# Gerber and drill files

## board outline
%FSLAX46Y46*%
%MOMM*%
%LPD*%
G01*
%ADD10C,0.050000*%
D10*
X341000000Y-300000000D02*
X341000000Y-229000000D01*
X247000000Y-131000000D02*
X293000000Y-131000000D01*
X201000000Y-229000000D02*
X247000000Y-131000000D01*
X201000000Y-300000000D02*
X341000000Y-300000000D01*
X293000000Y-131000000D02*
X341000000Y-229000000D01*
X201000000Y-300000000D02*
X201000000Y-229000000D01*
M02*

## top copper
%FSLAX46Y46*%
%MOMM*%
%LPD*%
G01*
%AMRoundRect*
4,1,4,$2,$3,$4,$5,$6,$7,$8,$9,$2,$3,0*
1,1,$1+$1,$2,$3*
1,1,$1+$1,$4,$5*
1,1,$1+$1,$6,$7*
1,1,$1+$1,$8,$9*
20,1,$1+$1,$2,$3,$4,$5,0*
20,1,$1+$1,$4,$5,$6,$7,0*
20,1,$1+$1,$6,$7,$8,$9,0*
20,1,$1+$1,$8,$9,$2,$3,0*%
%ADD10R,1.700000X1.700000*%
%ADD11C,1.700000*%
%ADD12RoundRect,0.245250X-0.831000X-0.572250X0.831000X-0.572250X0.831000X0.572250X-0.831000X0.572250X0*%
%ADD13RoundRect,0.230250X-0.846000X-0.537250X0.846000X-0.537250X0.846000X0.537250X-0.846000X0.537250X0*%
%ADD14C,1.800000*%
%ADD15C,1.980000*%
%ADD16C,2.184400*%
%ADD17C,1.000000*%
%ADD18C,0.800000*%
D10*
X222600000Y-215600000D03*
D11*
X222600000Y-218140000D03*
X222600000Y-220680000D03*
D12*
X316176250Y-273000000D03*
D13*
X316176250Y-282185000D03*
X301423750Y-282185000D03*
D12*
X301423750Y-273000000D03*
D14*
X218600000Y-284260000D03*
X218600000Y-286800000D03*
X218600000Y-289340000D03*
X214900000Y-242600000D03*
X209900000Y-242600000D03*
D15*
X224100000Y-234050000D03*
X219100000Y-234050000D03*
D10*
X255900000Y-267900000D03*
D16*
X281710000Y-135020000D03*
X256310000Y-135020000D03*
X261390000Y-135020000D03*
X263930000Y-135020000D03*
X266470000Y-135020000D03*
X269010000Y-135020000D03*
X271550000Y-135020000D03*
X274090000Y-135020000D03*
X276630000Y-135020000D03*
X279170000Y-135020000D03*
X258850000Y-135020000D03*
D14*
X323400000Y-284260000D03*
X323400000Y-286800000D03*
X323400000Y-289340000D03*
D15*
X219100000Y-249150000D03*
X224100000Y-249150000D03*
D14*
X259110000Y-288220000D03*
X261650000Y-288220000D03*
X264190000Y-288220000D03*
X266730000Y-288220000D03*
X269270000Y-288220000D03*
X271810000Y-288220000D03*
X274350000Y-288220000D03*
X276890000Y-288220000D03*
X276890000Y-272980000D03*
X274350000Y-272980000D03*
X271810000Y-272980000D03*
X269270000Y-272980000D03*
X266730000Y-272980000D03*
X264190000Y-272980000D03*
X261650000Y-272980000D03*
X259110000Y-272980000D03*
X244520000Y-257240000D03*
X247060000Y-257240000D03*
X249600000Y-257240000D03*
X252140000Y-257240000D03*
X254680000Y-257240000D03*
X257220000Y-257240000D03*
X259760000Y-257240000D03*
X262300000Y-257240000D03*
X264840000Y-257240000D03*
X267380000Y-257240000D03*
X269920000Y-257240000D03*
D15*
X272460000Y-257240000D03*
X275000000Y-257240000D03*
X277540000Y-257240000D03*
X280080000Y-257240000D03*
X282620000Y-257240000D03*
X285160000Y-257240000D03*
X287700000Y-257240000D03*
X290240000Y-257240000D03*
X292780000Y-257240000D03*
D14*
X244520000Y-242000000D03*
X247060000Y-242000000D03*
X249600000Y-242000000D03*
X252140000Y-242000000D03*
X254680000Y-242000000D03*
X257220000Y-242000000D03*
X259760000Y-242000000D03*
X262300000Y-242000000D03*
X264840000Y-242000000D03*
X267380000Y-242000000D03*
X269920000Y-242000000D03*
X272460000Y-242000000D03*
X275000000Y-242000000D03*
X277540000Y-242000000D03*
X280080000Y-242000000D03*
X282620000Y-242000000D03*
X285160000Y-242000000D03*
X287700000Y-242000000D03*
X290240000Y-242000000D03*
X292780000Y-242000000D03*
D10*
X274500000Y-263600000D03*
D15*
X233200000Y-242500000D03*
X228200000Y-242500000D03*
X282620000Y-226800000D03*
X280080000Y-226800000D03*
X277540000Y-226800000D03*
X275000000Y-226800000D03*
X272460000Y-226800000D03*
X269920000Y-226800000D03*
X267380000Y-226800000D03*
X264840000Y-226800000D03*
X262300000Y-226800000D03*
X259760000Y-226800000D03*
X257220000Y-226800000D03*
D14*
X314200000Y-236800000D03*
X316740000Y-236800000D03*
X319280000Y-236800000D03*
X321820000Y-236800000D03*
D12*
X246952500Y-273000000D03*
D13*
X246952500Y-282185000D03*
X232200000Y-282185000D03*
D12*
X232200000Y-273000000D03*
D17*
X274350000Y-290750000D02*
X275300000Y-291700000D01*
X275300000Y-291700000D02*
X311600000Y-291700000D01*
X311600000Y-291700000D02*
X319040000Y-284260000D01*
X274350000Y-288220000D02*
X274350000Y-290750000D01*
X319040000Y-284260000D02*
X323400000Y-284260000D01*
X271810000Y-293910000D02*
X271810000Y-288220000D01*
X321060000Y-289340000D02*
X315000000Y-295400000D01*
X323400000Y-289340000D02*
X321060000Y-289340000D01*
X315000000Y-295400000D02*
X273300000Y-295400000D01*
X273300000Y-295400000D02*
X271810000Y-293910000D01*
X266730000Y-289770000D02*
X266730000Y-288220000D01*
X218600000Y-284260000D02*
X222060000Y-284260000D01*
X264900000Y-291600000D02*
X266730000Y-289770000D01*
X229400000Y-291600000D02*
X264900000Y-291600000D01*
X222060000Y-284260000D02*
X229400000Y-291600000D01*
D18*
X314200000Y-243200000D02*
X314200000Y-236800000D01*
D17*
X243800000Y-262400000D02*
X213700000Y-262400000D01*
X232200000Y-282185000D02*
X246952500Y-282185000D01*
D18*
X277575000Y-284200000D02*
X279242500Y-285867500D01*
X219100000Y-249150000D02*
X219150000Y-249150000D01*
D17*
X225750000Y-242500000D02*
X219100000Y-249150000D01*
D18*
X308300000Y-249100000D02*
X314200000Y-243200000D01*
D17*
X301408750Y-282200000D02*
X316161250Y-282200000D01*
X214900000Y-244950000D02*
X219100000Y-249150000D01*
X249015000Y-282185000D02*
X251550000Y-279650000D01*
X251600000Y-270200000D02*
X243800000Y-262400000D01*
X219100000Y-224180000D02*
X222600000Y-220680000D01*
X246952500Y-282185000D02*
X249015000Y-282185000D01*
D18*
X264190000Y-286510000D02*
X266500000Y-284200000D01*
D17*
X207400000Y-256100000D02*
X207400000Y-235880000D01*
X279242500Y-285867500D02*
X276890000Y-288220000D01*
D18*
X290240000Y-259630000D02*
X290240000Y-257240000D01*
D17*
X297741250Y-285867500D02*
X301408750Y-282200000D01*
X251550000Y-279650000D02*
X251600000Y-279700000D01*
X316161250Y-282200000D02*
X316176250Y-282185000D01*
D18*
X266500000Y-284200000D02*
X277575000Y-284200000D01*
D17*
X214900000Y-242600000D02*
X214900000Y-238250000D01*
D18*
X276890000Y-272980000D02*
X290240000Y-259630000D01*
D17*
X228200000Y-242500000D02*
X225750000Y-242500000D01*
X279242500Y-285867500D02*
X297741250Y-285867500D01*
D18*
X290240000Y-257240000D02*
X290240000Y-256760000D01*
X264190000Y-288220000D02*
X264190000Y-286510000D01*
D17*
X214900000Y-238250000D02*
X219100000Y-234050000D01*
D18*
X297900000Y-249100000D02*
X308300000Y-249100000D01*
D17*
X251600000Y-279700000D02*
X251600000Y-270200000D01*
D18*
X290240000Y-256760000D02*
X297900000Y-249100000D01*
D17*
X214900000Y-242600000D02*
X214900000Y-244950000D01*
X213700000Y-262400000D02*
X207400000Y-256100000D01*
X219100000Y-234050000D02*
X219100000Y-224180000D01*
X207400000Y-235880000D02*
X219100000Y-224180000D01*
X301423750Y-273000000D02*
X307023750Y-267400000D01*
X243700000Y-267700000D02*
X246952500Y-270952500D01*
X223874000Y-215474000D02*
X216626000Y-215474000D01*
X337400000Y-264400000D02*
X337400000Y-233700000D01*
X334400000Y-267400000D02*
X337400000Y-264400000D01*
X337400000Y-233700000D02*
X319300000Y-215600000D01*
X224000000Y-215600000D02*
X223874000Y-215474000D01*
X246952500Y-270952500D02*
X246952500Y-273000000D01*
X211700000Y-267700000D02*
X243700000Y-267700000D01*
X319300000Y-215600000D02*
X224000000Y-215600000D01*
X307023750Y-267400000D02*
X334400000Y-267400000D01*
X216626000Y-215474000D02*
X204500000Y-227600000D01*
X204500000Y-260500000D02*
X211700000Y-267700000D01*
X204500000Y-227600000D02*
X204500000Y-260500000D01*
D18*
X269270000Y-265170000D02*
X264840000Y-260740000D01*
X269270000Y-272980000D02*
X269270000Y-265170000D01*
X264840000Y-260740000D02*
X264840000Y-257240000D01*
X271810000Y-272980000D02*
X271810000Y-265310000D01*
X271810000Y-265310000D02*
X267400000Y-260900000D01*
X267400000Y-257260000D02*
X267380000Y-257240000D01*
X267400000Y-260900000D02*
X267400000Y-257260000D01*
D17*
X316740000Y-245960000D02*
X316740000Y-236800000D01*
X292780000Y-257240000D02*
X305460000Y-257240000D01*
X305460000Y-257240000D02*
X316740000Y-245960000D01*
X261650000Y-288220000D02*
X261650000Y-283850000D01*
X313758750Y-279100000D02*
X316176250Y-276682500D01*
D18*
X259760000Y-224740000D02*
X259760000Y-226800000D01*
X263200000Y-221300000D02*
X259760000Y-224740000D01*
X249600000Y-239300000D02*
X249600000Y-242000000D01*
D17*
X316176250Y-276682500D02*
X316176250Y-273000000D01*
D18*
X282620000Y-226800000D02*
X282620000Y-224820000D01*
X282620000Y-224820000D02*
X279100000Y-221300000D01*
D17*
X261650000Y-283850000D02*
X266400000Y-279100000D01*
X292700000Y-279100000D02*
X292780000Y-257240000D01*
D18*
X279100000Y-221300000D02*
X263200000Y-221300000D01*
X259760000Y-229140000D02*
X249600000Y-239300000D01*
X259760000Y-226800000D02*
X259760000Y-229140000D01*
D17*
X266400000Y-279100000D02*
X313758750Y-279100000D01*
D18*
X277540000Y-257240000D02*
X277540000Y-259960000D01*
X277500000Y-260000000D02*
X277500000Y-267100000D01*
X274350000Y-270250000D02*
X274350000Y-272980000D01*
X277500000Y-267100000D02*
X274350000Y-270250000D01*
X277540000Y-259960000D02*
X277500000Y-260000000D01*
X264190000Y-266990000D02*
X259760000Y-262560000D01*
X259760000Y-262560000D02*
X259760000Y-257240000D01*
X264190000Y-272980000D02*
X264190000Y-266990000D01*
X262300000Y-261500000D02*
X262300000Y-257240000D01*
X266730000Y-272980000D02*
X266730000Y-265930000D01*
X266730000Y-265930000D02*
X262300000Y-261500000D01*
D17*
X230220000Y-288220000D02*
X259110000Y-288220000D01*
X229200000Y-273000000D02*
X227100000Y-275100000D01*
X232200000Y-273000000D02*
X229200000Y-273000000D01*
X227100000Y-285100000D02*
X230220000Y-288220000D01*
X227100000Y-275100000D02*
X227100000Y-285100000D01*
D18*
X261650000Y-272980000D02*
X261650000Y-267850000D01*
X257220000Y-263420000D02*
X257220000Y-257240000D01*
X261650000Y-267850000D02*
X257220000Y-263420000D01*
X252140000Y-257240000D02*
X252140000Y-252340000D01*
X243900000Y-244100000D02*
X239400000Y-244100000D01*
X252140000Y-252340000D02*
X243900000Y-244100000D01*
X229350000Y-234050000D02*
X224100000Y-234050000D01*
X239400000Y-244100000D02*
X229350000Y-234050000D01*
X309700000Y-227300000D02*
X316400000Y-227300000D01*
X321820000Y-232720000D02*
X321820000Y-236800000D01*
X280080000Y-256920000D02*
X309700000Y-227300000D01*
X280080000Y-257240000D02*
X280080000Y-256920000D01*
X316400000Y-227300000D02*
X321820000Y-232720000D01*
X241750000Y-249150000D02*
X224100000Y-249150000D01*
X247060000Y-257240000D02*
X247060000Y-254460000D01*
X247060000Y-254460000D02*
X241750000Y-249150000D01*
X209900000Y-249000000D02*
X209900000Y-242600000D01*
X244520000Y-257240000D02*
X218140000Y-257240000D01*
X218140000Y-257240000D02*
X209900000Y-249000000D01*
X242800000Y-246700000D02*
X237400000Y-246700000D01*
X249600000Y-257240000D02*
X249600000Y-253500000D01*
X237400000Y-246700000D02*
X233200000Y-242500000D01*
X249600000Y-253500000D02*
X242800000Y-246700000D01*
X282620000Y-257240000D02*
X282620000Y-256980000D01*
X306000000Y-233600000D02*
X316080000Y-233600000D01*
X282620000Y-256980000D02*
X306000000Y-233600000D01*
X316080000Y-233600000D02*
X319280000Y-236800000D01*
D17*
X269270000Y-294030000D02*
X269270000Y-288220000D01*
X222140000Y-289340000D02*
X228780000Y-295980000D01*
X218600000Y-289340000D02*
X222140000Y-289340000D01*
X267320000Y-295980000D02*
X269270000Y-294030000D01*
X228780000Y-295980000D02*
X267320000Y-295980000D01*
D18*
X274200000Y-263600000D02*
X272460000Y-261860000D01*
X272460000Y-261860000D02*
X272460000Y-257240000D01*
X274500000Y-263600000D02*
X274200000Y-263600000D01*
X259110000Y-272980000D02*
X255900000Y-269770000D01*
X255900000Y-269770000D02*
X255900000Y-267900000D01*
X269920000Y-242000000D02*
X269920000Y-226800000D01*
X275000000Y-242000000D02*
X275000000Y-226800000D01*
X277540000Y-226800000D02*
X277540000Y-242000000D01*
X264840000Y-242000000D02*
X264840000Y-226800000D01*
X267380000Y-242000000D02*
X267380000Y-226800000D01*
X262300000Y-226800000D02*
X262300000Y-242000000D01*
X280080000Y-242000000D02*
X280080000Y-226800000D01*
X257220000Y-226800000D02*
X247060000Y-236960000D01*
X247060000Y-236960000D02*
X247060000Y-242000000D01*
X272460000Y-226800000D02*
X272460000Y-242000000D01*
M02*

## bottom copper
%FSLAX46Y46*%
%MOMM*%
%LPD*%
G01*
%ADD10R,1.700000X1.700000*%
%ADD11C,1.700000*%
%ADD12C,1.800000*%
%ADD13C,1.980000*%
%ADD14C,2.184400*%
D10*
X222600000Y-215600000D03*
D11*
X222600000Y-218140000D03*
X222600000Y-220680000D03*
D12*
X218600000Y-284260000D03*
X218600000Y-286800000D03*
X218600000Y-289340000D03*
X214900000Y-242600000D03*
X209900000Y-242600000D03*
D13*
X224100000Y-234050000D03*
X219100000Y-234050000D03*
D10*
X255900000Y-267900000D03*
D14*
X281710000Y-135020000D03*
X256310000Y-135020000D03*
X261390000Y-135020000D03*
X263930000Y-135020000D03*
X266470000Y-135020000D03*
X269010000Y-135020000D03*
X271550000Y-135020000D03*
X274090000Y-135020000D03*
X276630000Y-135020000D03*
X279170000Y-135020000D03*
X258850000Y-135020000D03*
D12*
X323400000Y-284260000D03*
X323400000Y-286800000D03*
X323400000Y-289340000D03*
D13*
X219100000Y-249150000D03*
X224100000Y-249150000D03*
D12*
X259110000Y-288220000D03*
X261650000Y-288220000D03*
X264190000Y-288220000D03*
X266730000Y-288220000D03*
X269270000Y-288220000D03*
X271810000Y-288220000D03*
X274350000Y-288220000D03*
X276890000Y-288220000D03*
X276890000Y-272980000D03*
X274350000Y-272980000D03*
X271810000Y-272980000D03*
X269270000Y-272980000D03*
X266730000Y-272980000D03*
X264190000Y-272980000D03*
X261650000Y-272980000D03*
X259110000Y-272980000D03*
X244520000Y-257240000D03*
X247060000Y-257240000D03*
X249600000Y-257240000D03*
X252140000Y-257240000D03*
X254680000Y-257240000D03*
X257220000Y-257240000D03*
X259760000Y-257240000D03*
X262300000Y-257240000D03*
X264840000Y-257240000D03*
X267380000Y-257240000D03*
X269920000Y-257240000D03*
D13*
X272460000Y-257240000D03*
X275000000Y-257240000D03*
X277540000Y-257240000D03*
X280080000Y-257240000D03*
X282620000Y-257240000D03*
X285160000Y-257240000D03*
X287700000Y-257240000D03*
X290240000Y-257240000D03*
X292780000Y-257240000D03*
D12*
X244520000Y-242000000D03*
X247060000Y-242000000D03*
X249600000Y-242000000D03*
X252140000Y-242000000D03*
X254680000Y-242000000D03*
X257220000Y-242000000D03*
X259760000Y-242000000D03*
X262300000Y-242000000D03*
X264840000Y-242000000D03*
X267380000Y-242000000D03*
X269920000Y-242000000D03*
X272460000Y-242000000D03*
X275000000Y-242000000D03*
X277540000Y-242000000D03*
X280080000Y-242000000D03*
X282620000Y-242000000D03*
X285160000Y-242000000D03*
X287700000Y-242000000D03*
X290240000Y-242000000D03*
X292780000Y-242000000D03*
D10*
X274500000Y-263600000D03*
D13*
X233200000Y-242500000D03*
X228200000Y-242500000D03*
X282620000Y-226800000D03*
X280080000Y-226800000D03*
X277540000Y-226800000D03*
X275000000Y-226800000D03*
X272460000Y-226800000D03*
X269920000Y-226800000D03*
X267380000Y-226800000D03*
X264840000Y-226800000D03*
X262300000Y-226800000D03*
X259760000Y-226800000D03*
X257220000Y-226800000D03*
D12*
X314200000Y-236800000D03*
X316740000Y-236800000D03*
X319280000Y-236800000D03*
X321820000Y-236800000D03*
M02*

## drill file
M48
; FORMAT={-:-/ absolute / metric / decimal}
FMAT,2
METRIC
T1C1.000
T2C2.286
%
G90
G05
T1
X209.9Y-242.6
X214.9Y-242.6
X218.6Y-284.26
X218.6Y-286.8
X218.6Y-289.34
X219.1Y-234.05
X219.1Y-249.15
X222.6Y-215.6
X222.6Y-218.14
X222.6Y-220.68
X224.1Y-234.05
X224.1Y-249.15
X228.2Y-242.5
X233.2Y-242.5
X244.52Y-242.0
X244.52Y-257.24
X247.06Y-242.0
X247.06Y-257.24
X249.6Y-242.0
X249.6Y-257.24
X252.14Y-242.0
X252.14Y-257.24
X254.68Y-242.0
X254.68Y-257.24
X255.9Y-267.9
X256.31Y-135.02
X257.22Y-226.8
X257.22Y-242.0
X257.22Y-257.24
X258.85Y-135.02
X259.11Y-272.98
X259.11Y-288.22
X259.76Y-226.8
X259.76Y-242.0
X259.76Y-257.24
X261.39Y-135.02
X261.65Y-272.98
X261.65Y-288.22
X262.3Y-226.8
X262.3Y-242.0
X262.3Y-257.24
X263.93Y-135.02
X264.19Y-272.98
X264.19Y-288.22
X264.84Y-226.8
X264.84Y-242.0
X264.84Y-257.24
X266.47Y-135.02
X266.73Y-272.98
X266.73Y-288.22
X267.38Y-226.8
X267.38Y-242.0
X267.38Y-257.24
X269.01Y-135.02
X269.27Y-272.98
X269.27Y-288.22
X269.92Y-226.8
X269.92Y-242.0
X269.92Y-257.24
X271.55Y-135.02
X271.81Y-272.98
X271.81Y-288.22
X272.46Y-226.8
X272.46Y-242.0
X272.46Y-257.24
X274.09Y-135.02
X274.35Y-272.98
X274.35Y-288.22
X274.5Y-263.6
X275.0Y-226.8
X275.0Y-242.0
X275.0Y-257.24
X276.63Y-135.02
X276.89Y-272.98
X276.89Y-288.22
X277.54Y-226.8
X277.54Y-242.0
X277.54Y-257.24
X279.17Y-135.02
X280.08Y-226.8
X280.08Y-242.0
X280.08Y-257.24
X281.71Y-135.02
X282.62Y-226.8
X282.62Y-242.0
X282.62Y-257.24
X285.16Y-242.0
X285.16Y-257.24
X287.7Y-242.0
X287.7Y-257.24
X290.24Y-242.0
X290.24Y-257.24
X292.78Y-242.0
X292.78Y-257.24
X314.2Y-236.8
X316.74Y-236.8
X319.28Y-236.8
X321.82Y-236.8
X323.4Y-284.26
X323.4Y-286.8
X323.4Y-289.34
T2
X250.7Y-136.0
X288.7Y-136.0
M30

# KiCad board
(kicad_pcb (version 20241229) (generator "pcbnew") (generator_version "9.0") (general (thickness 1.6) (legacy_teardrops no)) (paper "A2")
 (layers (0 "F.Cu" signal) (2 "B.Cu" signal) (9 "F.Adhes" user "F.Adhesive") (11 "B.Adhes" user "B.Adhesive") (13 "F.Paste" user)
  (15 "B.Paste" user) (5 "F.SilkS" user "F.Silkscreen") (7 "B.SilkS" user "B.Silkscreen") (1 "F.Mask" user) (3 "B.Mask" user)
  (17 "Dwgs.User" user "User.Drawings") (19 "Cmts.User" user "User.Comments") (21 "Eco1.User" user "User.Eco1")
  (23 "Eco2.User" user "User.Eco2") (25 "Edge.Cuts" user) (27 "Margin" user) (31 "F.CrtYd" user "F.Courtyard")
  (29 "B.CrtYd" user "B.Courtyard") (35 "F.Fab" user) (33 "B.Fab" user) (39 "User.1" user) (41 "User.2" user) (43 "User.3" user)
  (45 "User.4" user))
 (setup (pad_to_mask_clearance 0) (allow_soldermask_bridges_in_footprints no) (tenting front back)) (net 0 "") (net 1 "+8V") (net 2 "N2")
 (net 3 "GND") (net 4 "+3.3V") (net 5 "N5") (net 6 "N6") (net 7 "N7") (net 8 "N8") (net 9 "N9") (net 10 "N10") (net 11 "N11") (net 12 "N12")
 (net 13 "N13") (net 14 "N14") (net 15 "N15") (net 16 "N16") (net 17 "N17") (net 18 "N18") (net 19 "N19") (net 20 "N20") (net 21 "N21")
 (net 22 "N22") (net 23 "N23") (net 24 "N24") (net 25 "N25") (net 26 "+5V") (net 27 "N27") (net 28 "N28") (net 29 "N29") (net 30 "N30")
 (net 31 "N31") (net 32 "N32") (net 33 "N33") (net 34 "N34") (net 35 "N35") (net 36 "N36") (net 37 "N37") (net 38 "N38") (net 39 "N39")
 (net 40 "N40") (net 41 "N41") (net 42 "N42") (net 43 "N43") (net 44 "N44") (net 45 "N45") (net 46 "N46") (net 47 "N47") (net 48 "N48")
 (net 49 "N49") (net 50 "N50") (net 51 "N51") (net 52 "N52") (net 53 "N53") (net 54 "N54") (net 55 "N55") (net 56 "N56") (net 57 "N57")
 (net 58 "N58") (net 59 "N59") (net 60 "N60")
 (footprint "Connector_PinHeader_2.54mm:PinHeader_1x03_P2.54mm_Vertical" (layer "F.Cu") (at 222.6 215.6)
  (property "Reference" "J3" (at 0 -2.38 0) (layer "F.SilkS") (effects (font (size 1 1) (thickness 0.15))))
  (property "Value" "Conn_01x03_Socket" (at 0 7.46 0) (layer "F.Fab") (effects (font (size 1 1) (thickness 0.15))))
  (pad "1" thru_hole rect (at 0 0) (size 1.7 1.7) (drill 1) (layers "*.Cu" "*.Mask") (remove_unused_layers no) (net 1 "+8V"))
  (pad "2" thru_hole circle (at 0 2.54) (size 1.7 1.7) (drill 1) (layers "*.Cu" "*.Mask") (remove_unused_layers no) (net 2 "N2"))
  (pad "3" thru_hole circle (at 0 5.08) (size 1.7 1.7) (drill 1) (layers "*.Cu" "*.Mask") (remove_unused_layers no) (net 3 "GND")))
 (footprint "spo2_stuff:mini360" (layer "F.Cu") (at 308.8 277.5175)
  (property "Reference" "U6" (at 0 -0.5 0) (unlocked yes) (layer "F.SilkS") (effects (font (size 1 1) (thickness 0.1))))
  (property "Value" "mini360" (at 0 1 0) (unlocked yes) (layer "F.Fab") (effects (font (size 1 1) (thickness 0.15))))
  (pad "1" smd roundrect (at 7.37625 -4.5175) (size 2.1525 1.635) (layers "F.Cu" "F.Mask" "F.Paste") (roundrect_rratio 0.15) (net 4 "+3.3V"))
  (pad "2" smd roundrect (at 7.37625 4.6675) (size 2.1525 1.535) (layers "F.Cu" "F.Mask" "F.Paste") (roundrect_rratio 0.15) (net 3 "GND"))
  (pad "3" smd roundrect (at -7.37625 4.6675) (size 2.1525 1.535) (layers "F.Cu" "F.Mask" "F.Paste") (roundrect_rratio 0.15) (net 3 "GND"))
  (pad "4" smd roundrect (at -7.37625 -4.5175) (size 2.1525 1.635) (layers "F.Cu" "F.Mask" "F.Paste") (roundrect_rratio 0.15) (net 1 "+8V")))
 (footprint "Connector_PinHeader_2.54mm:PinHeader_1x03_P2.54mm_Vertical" (layer "F.Cu") (at 218.6 284.26)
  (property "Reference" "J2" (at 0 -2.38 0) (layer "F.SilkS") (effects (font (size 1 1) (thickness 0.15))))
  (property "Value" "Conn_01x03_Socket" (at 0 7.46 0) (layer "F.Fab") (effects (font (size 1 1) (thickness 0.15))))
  (pad "1" thru_hole circle (at 0 0) (size 1.8 1.8) (drill 1) (layers "*.Cu" "*.Mask") (remove_unused_layers no) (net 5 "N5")
   (solder_mask_margin 0.102))
  (pad "2" thru_hole circle (at 0 2.54) (size 1.8 1.8) (drill 1) (layers "*.Cu" "*.Mask") (remove_unused_layers no) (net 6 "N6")
   (solder_mask_margin 0.102))
  (pad "3" thru_hole circle (at 0 5.08) (size 1.8 1.8) (drill 1) (layers "*.Cu" "*.Mask") (remove_unused_layers no) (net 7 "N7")
   (solder_mask_margin 0.102)))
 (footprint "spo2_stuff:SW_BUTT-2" (layer "F.Cu") (at 212.4 242.6 180)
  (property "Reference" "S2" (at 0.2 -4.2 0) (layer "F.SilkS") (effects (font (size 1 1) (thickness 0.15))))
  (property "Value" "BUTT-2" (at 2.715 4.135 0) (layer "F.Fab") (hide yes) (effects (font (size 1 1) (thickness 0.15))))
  (pad "1" thru_hole circle (at -2.5 0 180) (size 1.8 1.8) (drill 1) (layers "*.Cu" "*.Mask") (remove_unused_layers no) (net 3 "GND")
   (solder_mask_margin 0.102))
  (pad "2" thru_hole circle (at 2.5 0 180) (size 1.8 1.8) (drill 1) (layers "*.Cu" "*.Mask") (remove_unused_layers no) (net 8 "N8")
   (solder_mask_margin 0.102)))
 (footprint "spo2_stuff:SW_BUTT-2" (layer "F.Cu") (at 221.6 234.05 180)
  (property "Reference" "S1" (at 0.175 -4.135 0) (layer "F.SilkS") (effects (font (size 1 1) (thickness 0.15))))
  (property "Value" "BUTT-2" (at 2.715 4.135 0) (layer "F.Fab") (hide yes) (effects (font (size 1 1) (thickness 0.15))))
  (pad "1" thru_hole circle (at -2.5 0 180) (size 1.98 1.98) (drill 1) (layers "*.Cu" "*.Mask") (remove_unused_layers no) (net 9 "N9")
   (solder_mask_margin 0.102))
  (pad "2" thru_hole circle (at 2.5 0 180) (size 1.98 1.98) (drill 1) (layers "*.Cu" "*.Mask") (remove_unused_layers no) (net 3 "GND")
   (solder_mask_margin 0.102)))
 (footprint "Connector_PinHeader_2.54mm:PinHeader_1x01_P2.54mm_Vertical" (layer "F.Cu") (at 255.9 267.9)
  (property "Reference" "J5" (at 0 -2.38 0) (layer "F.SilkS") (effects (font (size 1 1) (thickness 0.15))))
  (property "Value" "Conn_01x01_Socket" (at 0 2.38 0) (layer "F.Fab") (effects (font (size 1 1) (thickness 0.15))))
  (pad "1" thru_hole rect (at 0 0) (size 1.7 1.7) (drill 1) (layers "*.Cu" "*.Mask") (remove_unused_layers no) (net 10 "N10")))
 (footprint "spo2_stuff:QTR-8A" (layer "F.Cu") (at 289.35 133.75)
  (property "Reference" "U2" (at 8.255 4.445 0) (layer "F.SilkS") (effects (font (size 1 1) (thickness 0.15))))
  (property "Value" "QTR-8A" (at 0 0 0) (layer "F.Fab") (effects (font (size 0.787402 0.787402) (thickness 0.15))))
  (pad "" np_thru_hole circle (at -38.65 2.25) (size 2.286 2.286) (drill 2.286) (layers "*.Cu" "*.Mask"))
  (pad "" np_thru_hole circle (at -0.65 2.25) (size 2.286 2.286) (drill 2.286) (layers "*.Cu" "*.Mask"))
  (pad "3V3" thru_hole circle (at -7.64 1.27) (size 2.1844 2.1844) (drill 1) (layers "*.Cu" "*.Mask") (remove_unused_layers no)
   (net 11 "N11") (solder_mask_margin 0.102))
  (pad "GND" thru_hole circle (at -33.04 1.27) (size 2.1844 2.1844) (drill 1) (layers "*.Cu" "*.Mask") (remove_unused_layers no)
   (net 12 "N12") (solder_mask_margin 0.102))
  (pad "LED1" thru_hole circle (at -27.96 1.27) (size 2.1844 2.1844) (drill 1) (layers "*.Cu" "*.Mask") (remove_unused_layers no)
   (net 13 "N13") (solder_mask_margin 0.102))
  (pad "LED2" thru_hole circle (at -25.42 1.27) (size 2.1844 2.1844) (drill 1) (layers "*.Cu" "*.Mask") (remove_unused_layers no)
   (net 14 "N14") (solder_mask_margin 0.102))
  (pad "LED3" thru_hole circle (at -22.88 1.27) (size 2.1844 2.1844) (drill 1) (layers "*.Cu" "*.Mask") (remove_unused_layers no)
   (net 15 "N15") (solder_mask_margin 0.102))
  (pad "LED4" thru_hole circle (at -20.34 1.27) (size 2.1844 2.1844) (drill 1) (layers "*.Cu" "*.Mask") (remove_unused_layers no)
   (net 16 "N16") (solder_mask_margin 0.102))
  (pad "LED5" thru_hole circle (at -17.8 1.27) (size 2.1844 2.1844) (drill 1) (layers "*.Cu" "*.Mask") (remove_unused_layers no)
   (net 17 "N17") (solder_mask_margin 0.102))
  (pad "LED6" thru_hole circle (at -15.26 1.27) (size 2.1844 2.1844) (drill 1) (layers "*.Cu" "*.Mask") (remove_unused_layers no)
   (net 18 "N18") (solder_mask_margin 0.102))
  (pad "LED7" thru_hole circle (at -12.72 1.27) (size 2.1844 2.1844) (drill 1) (layers "*.Cu" "*.Mask") (remove_unused_layers no)
   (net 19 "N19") (solder_mask_margin 0.102))
  (pad "LED8" thru_hole circle (at -10.18 1.27) (size 2.1844 2.1844) (drill 1) (layers "*.Cu" "*.Mask") (remove_unused_layers no)
   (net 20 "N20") (solder_mask_margin 0.102))
  (pad "LED_ON" thru_hole circle (at -30.5 1.27) (size 2.1844 2.1844) (drill 1) (layers "*.Cu" "*.Mask") (remove_unused_layers no)
   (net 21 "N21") (solder_mask_margin 0.102)))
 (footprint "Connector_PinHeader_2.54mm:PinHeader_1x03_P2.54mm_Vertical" (layer "F.Cu") (at 323.4 284.26)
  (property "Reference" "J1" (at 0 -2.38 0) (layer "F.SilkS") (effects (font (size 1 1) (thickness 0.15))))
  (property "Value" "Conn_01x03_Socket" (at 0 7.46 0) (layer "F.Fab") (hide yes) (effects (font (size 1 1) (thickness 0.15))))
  (pad "1" thru_hole circle (at 0 0) (size 1.8 1.8) (drill 1) (layers "*.Cu" "*.Mask") (remove_unused_layers no) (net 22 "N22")
   (solder_mask_margin 0.102))
  (pad "2" thru_hole circle (at 0 2.54) (size 1.8 1.8) (drill 1) (layers "*.Cu" "*.Mask") (remove_unused_layers no) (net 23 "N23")
   (solder_mask_margin 0.102))
  (pad "3" thru_hole circle (at 0 5.08) (size 1.8 1.8) (drill 1) (layers "*.Cu" "*.Mask") (remove_unused_layers no) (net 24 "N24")
   (solder_mask_margin 0.102)))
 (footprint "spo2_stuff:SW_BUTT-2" (layer "F.Cu") (at 221.6 249.15)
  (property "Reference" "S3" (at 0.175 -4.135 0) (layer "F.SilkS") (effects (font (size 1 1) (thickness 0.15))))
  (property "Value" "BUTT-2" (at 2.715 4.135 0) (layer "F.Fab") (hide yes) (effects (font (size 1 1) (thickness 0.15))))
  (pad "1" thru_hole circle (at -2.5 0) (size 1.98 1.98) (drill 1) (layers "*.Cu" "*.Mask") (remove_unused_layers no) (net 3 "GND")
   (solder_mask_margin 0.102))
  (pad "2" thru_hole circle (at 2.5 0) (size 1.98 1.98) (drill 1) (layers "*.Cu" "*.Mask") (remove_unused_layers no) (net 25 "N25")
   (solder_mask_margin 0.102)))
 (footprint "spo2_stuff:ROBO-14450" (layer "F.Cu") (at 268 280.6 90)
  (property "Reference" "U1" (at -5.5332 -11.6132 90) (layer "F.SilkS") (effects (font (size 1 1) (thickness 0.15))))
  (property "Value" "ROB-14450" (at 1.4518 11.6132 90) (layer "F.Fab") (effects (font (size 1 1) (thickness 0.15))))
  (pad "1" thru_hole circle (at -7.62 -8.89 90) (size 1.8 1.8) (drill 1) (layers "*.Cu" "*.Mask") (remove_unused_layers no) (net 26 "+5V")
   (solder_mask_margin 0.102))
  (pad "2" thru_hole circle (at -7.62 -6.35 90) (size 1.8 1.8) (drill 1) (layers "*.Cu" "*.Mask") (remove_unused_layers no) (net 4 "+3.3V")
   (solder_mask_margin 0.102))
  (pad "3" thru_hole circle (at -7.62 -3.81 90) (size 1.8 1.8) (drill 1) (layers "*.Cu" "*.Mask") (remove_unused_layers no) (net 3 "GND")
   (solder_mask_margin 0.102))
  (pad "4" thru_hole circle (at -7.62 -1.27 90) (size 1.8 1.8) (drill 1) (layers "*.Cu" "*.Mask") (remove_unused_layers no) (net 5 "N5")
   (solder_mask_margin 0.102))
  (pad "5" thru_hole circle (at -7.62 1.27 90) (size 1.8 1.8) (drill 1) (layers "*.Cu" "*.Mask") (remove_unused_layers no) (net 7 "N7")
   (solder_mask_margin 0.102))
  (pad "6" thru_hole circle (at -7.62 3.81 90) (size 1.8 1.8) (drill 1) (layers "*.Cu" "*.Mask") (remove_unused_layers no) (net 24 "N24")
   (solder_mask_margin 0.102))
  (pad "7" thru_hole circle (at -7.62 6.35 90) (size 1.8 1.8) (drill 1) (layers "*.Cu" "*.Mask") (remove_unused_layers no) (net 22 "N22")
   (solder_mask_margin 0.102))
  (pad "8" thru_hole circle (at -7.62 8.89 90) (size 1.8 1.8) (drill 1) (layers "*.Cu" "*.Mask") (remove_unused_layers no) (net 3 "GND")
   (solder_mask_margin 0.102))
  (pad "9" thru_hole circle (at 7.62 8.89 90) (size 1.8 1.8) (drill 1) (layers "*.Cu" "*.Mask") (remove_unused_layers no) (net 3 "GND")
   (solder_mask_margin 0.102))
  (pad "10" thru_hole circle (at 7.62 6.35 90) (size 1.8 1.8) (drill 1) (layers "*.Cu" "*.Mask") (remove_unused_layers no) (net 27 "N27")
   (solder_mask_margin 0.102))
  (pad "11" thru_hole circle (at 7.62 3.81 90) (size 1.8 1.8) (drill 1) (layers "*.Cu" "*.Mask") (remove_unused_layers no) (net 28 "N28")
   (solder_mask_margin 0.102))
  (pad "12" thru_hole circle (at 7.62 1.27 90) (size 1.8 1.8) (drill 1) (layers "*.Cu" "*.Mask") (remove_unused_layers no) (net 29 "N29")
   (solder_mask_margin 0.102))
  (pad "13" thru_hole circle (at 7.62 -1.27 90) (size 1.8 1.8) (drill 1) (layers "*.Cu" "*.Mask") (remove_unused_layers no) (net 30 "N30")
   (solder_mask_margin 0.102))
  (pad "14" thru_hole circle (at 7.62 -3.81 90) (size 1.8 1.8) (drill 1) (layers "*.Cu" "*.Mask") (remove_unused_layers no) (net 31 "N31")
   (solder_mask_margin 0.102))
  (pad "15" thru_hole circle (at 7.62 -6.35 90) (size 1.8 1.8) (drill 1) (layers "*.Cu" "*.Mask") (remove_unused_layers no) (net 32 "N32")
   (solder_mask_margin 0.102))
  (pad "16" thru_hole circle (at 7.62 -8.89 90) (size 1.8 1.8) (drill 1) (layers "*.Cu" "*.Mask") (remove_unused_layers no) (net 10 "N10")
   (solder_mask_margin 0.102)))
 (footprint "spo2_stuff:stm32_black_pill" (layer "F.Cu") (at 295.1 260.15 90)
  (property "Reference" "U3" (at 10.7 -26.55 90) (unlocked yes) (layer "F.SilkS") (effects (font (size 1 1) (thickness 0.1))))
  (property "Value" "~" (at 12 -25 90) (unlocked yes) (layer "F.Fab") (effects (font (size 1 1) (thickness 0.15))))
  (pad "1" thru_hole circle (at 2.91 -50.58 90) (size 1.8 1.8) (drill 1) (layers "*.Cu" "*.Mask") (remove_unused_layers no) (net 8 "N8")
   (solder_mask_margin 0.102))
  (pad "2" thru_hole circle (at 2.91 -48.04 90) (size 1.8 1.8) (drill 1) (layers "*.Cu" "*.Mask") (remove_unused_layers no) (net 25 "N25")
   (solder_mask_margin 0.102))
  (pad "3" thru_hole circle (at 2.91 -45.5 90) (size 1.8 1.8) (drill 1) (layers "*.Cu" "*.Mask") (remove_unused_layers no) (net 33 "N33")
   (solder_mask_margin 0.102))
  (pad "4" thru_hole circle (at 2.91 -42.96 90) (size 1.8 1.8) (drill 1) (layers "*.Cu" "*.Mask") (remove_unused_layers no) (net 9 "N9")
   (solder_mask_margin 0.102))
  (pad "5" thru_hole circle (at 2.91 -40.42 90) (size 1.8 1.8) (drill 1) (layers "*.Cu" "*.Mask") (remove_unused_layers no) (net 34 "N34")
   (solder_mask_margin 0.102))
  (pad "6" thru_hole circle (at 2.91 -37.88 90) (size 1.8 1.8) (drill 1) (layers "*.Cu" "*.Mask") (remove_unused_layers no) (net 32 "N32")
   (solder_mask_margin 0.102))
  (pad "7" thru_hole circle (at 2.91 -35.34 90) (size 1.8 1.8) (drill 1) (layers "*.Cu" "*.Mask") (remove_unused_layers no) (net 31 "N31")
   (solder_mask_margin 0.102))
  (pad "8" thru_hole circle (at 2.91 -32.8 90) (size 1.8 1.8) (drill 1) (layers "*.Cu" "*.Mask") (remove_unused_layers no) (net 30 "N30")
   (solder_mask_margin 0.102))
  (pad "9" thru_hole circle (at 2.91 -30.26 90) (size 1.8 1.8) (drill 1) (layers "*.Cu" "*.Mask") (remove_unused_layers no) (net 29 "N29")
   (solder_mask_margin 0.102))
  (pad "10" thru_hole circle (at 2.91 -27.72 90) (size 1.8 1.8) (drill 1) (layers "*.Cu" "*.Mask") (remove_unused_layers no) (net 28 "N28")
   (solder_mask_margin 0.102))
  (pad "11" thru_hole circle (at 2.91 -25.18 90) (size 1.8 1.8) (drill 1) (layers "*.Cu" "*.Mask") (remove_unused_layers no) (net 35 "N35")
   (solder_mask_margin 0.102))
  (pad "12" thru_hole circle (at 2.91 -22.64 90) (size 1.98 1.98) (drill 1) (layers "*.Cu" "*.Mask") (remove_unused_layers no)
   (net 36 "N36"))
  (pad "13" thru_hole circle (at 2.91 -20.1 90) (size 1.98 1.98) (drill 1) (layers "*.Cu" "*.Mask") (remove_unused_layers no) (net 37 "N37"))
  (pad "14" thru_hole circle (at 2.91 -17.56 90) (size 1.98 1.98) (drill 1) (layers "*.Cu" "*.Mask") (remove_unused_layers no)
   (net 27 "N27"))
  (pad "15" thru_hole circle (at 2.91 -15.02 90) (size 1.98 1.98) (drill 1) (layers "*.Cu" "*.Mask") (remove_unused_layers no)
   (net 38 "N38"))
  (pad "16" thru_hole circle (at 2.91 -12.48 90) (size 1.98 1.98) (drill 1) (layers "*.Cu" "*.Mask") (remove_unused_layers no)
   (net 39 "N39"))
  (pad "17" thru_hole circle (at 2.91 -9.94 90) (size 1.98 1.98) (drill 1) (layers "*.Cu" "*.Mask") (remove_unused_layers no) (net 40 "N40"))
  (pad "18" thru_hole circle (at 2.91 -7.4 90) (size 1.98 1.98) (drill 1) (layers "*.Cu" "*.Mask") (remove_unused_layers no) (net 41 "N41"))
  (pad "19" thru_hole circle (at 2.91 -4.86 90) (size 1.98 1.98) (drill 1) (layers "*.Cu" "*.Mask") (remove_unused_layers no) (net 3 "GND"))
  (pad "20" thru_hole circle (at 2.91 -2.32 90) (size 1.98 1.98) (drill 1) (layers "*.Cu" "*.Mask") (remove_unused_layers no)
   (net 4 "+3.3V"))
  (pad "21" thru_hole circle (at 18.15 -50.58 90) (size 1.8 1.8) (drill 1) (layers "*.Cu" "*.Mask") (remove_unused_layers no) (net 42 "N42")
   (solder_mask_margin 0.102))
  (pad "22" thru_hole circle (at 18.15 -48.04 90) (size 1.8 1.8) (drill 1) (layers "*.Cu" "*.Mask") (remove_unused_layers no) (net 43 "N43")
   (solder_mask_margin 0.102))
  (pad "23" thru_hole circle (at 18.15 -45.5 90) (size 1.8 1.8) (drill 1) (layers "*.Cu" "*.Mask") (remove_unused_layers no) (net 4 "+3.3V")
   (solder_mask_margin 0.102))
  (pad "24" thru_hole circle (at 18.15 -42.96 90) (size 1.8 1.8) (drill 1) (layers "*.Cu" "*.Mask") (remove_unused_layers no) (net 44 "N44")
   (solder_mask_margin 0.102))
  (pad "25" thru_hole circle (at 18.15 -40.42 90) (size 1.8 1.8) (drill 1) (layers "*.Cu" "*.Mask") (remove_unused_layers no) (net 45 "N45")
   (solder_mask_margin 0.102))
  (pad "26" thru_hole circle (at 18.15 -37.88 90) (size 1.8 1.8) (drill 1) (layers "*.Cu" "*.Mask") (remove_unused_layers no) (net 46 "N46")
   (solder_mask_margin 0.102))
  (pad "27" thru_hole circle (at 18.15 -35.34 90) (size 1.8 1.8) (drill 1) (layers "*.Cu" "*.Mask") (remove_unused_layers no) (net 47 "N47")
   (solder_mask_margin 0.102))
  (pad "28" thru_hole circle (at 18.15 -32.8 90) (size 1.8 1.8) (drill 1) (layers "*.Cu" "*.Mask") (remove_unused_layers no) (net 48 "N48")
   (solder_mask_margin 0.102))
  (pad "29" thru_hole circle (at 18.15 -30.26 90) (size 1.8 1.8) (drill 1) (layers "*.Cu" "*.Mask") (remove_unused_layers no) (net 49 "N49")
   (solder_mask_margin 0.102))
  (pad "30" thru_hole circle (at 18.15 -27.72 90) (size 1.8 1.8) (drill 1) (layers "*.Cu" "*.Mask") (remove_unused_layers no) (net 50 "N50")
   (solder_mask_margin 0.102))
  (pad "31" thru_hole circle (at 18.15 -25.18 90) (size 1.8 1.8) (drill 1) (layers "*.Cu" "*.Mask") (remove_unused_layers no) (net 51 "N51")
   (solder_mask_margin 0.102))
  (pad "32" thru_hole circle (at 18.15 -22.64 90) (size 1.8 1.8) (drill 1) (layers "*.Cu" "*.Mask") (remove_unused_layers no) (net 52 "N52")
   (solder_mask_margin 0.102))
  (pad "33" thru_hole circle (at 18.15 -20.1 90) (size 1.8 1.8) (drill 1) (layers "*.Cu" "*.Mask") (remove_unused_layers no) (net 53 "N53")
   (solder_mask_margin 0.102))
  (pad "34" thru_hole circle (at 18.15 -17.56 90) (size 1.8 1.8) (drill 1) (layers "*.Cu" "*.Mask") (remove_unused_layers no) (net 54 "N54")
   (solder_mask_margin 0.102))
  (pad "35" thru_hole circle (at 18.15 -15.02 90) (size 1.8 1.8) (drill 1) (layers "*.Cu" "*.Mask") (remove_unused_layers no) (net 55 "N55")
   (solder_mask_margin 0.102))
  (pad "36" thru_hole circle (at 18.15 -12.48 90) (size 1.8 1.8) (drill 1) (layers "*.Cu" "*.Mask") (remove_unused_layers no) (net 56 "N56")
   (solder_mask_margin 0.102))
  (pad "37" thru_hole circle (at 18.15 -9.94 90) (size 1.8 1.8) (drill 1) (layers "*.Cu" "*.Mask") (remove_unused_layers no) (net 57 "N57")
   (solder_mask_margin 0.102))
  (pad "38" thru_hole circle (at 18.15 -7.4 90) (size 1.8 1.8) (drill 1) (layers "*.Cu" "*.Mask") (remove_unused_layers no) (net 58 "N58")
   (solder_mask_margin 0.102))
  (pad "39" thru_hole circle (at 18.15 -4.86 90) (size 1.8 1.8) (drill 1) (layers "*.Cu" "*.Mask") (remove_unused_layers no) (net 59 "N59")
   (solder_mask_margin 0.102))
  (pad "40" thru_hole circle (at 18.15 -2.32 90) (size 1.8 1.8) (drill 1) (layers "*.Cu" "*.Mask") (remove_unused_layers no) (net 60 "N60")
   (solder_mask_margin 0.102)))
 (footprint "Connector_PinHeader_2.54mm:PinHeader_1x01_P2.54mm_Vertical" (layer "F.Cu") (at 274.5 263.6)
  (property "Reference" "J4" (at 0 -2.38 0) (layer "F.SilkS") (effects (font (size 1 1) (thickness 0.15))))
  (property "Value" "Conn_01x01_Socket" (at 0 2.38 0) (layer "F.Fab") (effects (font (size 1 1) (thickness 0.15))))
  (pad "1" thru_hole rect (at 0 0) (size 1.7 1.7) (drill 1) (layers "*.Cu" "*.Mask") (remove_unused_layers no) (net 36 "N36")))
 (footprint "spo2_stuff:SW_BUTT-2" (layer "F.Cu") (at 230.7 242.5 180)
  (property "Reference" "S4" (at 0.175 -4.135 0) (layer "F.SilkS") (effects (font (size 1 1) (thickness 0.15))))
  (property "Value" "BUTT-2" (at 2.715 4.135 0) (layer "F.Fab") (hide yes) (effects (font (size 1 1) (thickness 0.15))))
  (pad "1" thru_hole circle (at -2.5 0 180) (size 1.98 1.98) (drill 1) (layers "*.Cu" "*.Mask") (remove_unused_layers no) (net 33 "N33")
   (solder_mask_margin 0.102))
  (pad "2" thru_hole circle (at 2.5 0 180) (size 1.98 1.98) (drill 1) (layers "*.Cu" "*.Mask") (remove_unused_layers no) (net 3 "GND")
   (solder_mask_margin 0.102)))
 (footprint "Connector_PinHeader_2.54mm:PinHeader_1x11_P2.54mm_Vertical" (layer "F.Cu") (at 282.62 226.8 -90)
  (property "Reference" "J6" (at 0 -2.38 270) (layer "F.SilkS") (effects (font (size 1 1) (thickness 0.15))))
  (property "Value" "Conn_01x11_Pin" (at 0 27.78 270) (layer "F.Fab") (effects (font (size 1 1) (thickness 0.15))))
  (pad "1" thru_hole circle (at 0 0 270) (size 1.98 1.98) (drill 1) (layers "*.Cu" "*.Mask") (remove_unused_layers no) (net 4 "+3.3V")
   (solder_mask_margin 0.102))
  (pad "2" thru_hole circle (at 0 2.54 270) (size 1.98 1.98) (drill 1) (layers "*.Cu" "*.Mask") (remove_unused_layers no) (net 55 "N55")
   (solder_mask_margin 0.102))
  (pad "3" thru_hole circle (at 0 5.08 270) (size 1.98 1.98) (drill 1) (layers "*.Cu" "*.Mask") (remove_unused_layers no) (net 54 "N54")
   (solder_mask_margin 0.102))
  (pad "4" thru_hole circle (at 0 7.62 270) (size 1.98 1.98) (drill 1) (layers "*.Cu" "*.Mask") (remove_unused_layers no) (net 53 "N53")
   (solder_mask_margin 0.102))
  (pad "5" thru_hole circle (at 0 10.16 270) (size 1.98 1.98) (drill 1) (layers "*.Cu" "*.Mask") (remove_unused_layers no) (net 52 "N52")
   (solder_mask_margin 0.102))
  (pad "6" thru_hole circle (at 0 12.7 270) (size 1.98 1.98) (drill 1) (layers "*.Cu" "*.Mask") (remove_unused_layers no) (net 51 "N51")
   (solder_mask_margin 0.102))
  (pad "7" thru_hole circle (at 0 15.24 270) (size 1.98 1.98) (drill 1) (layers "*.Cu" "*.Mask") (remove_unused_layers no) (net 50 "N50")
   (solder_mask_margin 0.102))
  (pad "8" thru_hole circle (at 0 17.78 270) (size 1.98 1.98) (drill 1) (layers "*.Cu" "*.Mask") (remove_unused_layers no) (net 49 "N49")
   (solder_mask_margin 0.102))
  (pad "9" thru_hole circle (at 0 20.32 270) (size 1.98 1.98) (drill 1) (layers "*.Cu" "*.Mask") (remove_unused_layers no) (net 48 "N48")
   (solder_mask_margin 0.102))
  (pad "10" thru_hole circle (at 0 22.86 270) (size 1.98 1.98) (drill 1) (layers "*.Cu" "*.Mask") (remove_unused_layers no) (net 4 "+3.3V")
   (solder_mask_margin 0.102))
  (pad "11" thru_hole circle (at 0 25.4 270) (size 1.98 1.98) (drill 1) (layers "*.Cu" "*.Mask") (remove_unused_layers no) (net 43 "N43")
   (solder_mask_margin 0.102)))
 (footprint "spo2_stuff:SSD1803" (layer "F.Cu") (at 318.01 249.5)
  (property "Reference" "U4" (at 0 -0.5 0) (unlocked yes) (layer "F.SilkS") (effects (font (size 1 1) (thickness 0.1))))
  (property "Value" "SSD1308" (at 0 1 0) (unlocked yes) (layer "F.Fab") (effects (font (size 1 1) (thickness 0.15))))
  (pad "1" thru_hole circle (at -3.81 -12.7) (size 1.8 1.8) (drill 1) (layers "*.Cu" "*.Mask") (remove_unused_layers no) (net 3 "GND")
   (solder_mask_margin 0.102))
  (pad "2" thru_hole circle (at -1.27 -12.7) (size 1.8 1.8) (drill 1) (layers "*.Cu" "*.Mask") (remove_unused_layers no) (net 4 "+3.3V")
   (solder_mask_margin 0.102))
  (pad "3" thru_hole circle (at 1.27 -12.7) (size 1.8 1.8) (drill 1) (layers "*.Cu" "*.Mask") (remove_unused_layers no) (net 39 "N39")
   (solder_mask_margin 0.102))
  (pad "4" thru_hole circle (at 3.81 -12.7) (size 1.8 1.8) (drill 1) (layers "*.Cu" "*.Mask") (remove_unused_layers no) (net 38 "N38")
   (solder_mask_margin 0.102))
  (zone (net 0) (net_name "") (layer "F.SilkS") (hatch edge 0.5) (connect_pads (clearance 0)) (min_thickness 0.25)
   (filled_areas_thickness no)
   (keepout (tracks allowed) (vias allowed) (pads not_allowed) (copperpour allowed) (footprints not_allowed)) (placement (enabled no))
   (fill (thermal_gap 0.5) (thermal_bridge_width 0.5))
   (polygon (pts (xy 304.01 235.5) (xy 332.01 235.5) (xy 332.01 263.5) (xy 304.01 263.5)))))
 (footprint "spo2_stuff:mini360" (layer "F.Cu") (at 239.57625 277.5175)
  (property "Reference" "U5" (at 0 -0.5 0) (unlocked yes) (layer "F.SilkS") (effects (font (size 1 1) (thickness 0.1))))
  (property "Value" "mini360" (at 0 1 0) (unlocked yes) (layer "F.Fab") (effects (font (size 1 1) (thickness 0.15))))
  (pad "1" smd roundrect (at 7.37625 -4.5175) (size 2.1525 1.635) (layers "F.Cu" "F.Mask" "F.Paste") (roundrect_rratio 0.15) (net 1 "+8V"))
  (pad "2" smd roundrect (at 7.37625 4.6675) (size 2.1525 1.535) (layers "F.Cu" "F.Mask" "F.Paste") (roundrect_rratio 0.15) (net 3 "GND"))
  (pad "3" smd roundrect (at -7.37625 4.6675) (size 2.1525 1.535) (layers "F.Cu" "F.Mask" "F.Paste") (roundrect_rratio 0.15) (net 3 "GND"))
  (pad "4" smd roundrect (at -7.37625 -4.5175) (size 2.1525 1.635) (layers "F.Cu" "F.Mask" "F.Paste") (roundrect_rratio 0.15) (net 26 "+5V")))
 (gr_line (start 341 300) (end 341 229) (stroke (width 0.05) (type solid)) (layer "Edge.Cuts"))
 (gr_line (start 247 131) (end 293 131) (stroke (width 0.05) (type solid)) (layer "Edge.Cuts"))
 (gr_line (start 201 229) (end 247 131) (stroke (width 0.05) (type default)) (layer "Edge.Cuts"))
 (gr_line (start 201 300) (end 341 300) (stroke (width 0.05) (type solid)) (layer "Edge.Cuts"))
 (gr_line (start 293 131) (end 341 229) (stroke (width 0.05) (type default)) (layer "Edge.Cuts"))
 (gr_line (start 201 300) (end 201 229) (stroke (width 0.05) (type solid)) (layer "Edge.Cuts"))
 (segment (start 274.35 290.75) (end 275.3 291.7) (width 1) (layer "F.Cu") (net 22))
 (segment (start 275.3 291.7) (end 311.6 291.7) (width 1) (layer "F.Cu") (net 22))
 (segment (start 311.6 291.7) (end 319.04 284.26) (width 1) (layer "F.Cu") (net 22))
 (segment (start 274.35 288.22) (end 274.35 290.75) (width 1) (layer "F.Cu") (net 22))
 (segment (start 319.04 284.26) (end 323.4 284.26) (width 1) (layer "F.Cu") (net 22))
 (segment (start 271.81 293.91) (end 271.81 288.22) (width 1) (layer "F.Cu") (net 24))
 (segment (start 321.06 289.34) (end 315 295.4) (width 1) (layer "F.Cu") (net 24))
 (segment (start 323.4 289.34) (end 321.06 289.34) (width 1) (layer "F.Cu") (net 24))
 (segment (start 315 295.4) (end 273.3 295.4) (width 1) (layer "F.Cu") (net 24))
 (segment (start 273.3 295.4) (end 271.81 293.91) (width 1) (layer "F.Cu") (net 24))
 (segment (start 266.73 289.77) (end 266.73 288.22) (width 1) (layer "F.Cu") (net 5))
 (segment (start 218.6 284.26) (end 222.06 284.26) (width 1) (layer "F.Cu") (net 5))
 (segment (start 264.9 291.6) (end 266.73 289.77) (width 1) (layer "F.Cu") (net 5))
 (segment (start 229.4 291.6) (end 264.9 291.6) (width 1) (layer "F.Cu") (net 5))
 (segment (start 222.06 284.26) (end 229.4 291.6) (width 1) (layer "F.Cu") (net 5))
 (segment (start 314.2 243.2) (end 314.2 236.8) (width 0.8) (layer "F.Cu") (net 3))
 (segment (start 243.8 262.4) (end 213.7 262.4) (width 1) (layer "F.Cu") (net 3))
 (segment (start 232.2 282.185) (end 246.9525 282.185) (width 1) (layer "F.Cu") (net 3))
 (segment (start 277.575 284.2) (end 279.2425 285.8675) (width 0.8) (layer "F.Cu") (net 3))
 (segment (start 219.1 249.15) (end 219.15 249.15) (width 0.8) (layer "F.Cu") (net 3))
 (segment (start 225.75 242.5) (end 219.1 249.15) (width 1) (layer "F.Cu") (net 3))
 (segment (start 308.3 249.1) (end 314.2 243.2) (width 0.8) (layer "F.Cu") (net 3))
 (segment (start 301.40875 282.2) (end 316.16125 282.2) (width 1) (layer "F.Cu") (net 3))
 (segment (start 214.9 244.95) (end 219.1 249.15) (width 1) (layer "F.Cu") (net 3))
 (segment (start 249.015 282.185) (end 251.55 279.65) (width 1) (layer "F.Cu") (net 3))
 (segment (start 251.6 270.2) (end 243.8 262.4) (width 1) (layer "F.Cu") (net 3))
 (segment (start 219.1 224.18) (end 222.6 220.68) (width 1) (layer "F.Cu") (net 3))
 (segment (start 246.9525 282.185) (end 249.015 282.185) (width 1) (layer "F.Cu") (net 3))
 (segment (start 264.19 286.51) (end 266.5 284.2) (width 0.8) (layer "F.Cu") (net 3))
 (segment (start 207.4 256.1) (end 207.4 235.88) (width 1) (layer "F.Cu") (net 3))
 (segment (start 279.2425 285.8675) (end 276.89 288.22) (width 1) (layer "F.Cu") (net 3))
 (segment (start 290.24 259.63) (end 290.24 257.24) (width 0.8) (layer "F.Cu") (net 3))
 (segment (start 297.74125 285.8675) (end 301.40875 282.2) (width 1) (layer "F.Cu") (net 3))
 (segment (start 251.55 279.65) (end 251.6 279.7) (width 1) (layer "F.Cu") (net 3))
 (segment (start 316.16125 282.2) (end 316.17625 282.185) (width 1) (layer "F.Cu") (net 3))
 (segment (start 266.5 284.2) (end 277.575 284.2) (width 0.8) (layer "F.Cu") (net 3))
 (segment (start 214.9 242.6) (end 214.9 238.25) (width 1) (layer "F.Cu") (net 3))
 (segment (start 276.89 272.98) (end 290.24 259.63) (width 0.8) (layer "F.Cu") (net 3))
 (segment (start 228.2 242.5) (end 225.75 242.5) (width 1) (layer "F.Cu") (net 3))
 (segment (start 279.2425 285.8675) (end 297.74125 285.8675) (width 1) (layer "F.Cu") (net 3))
 (segment (start 290.24 257.24) (end 290.24 256.76) (width 0.8) (layer "F.Cu") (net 3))
 (segment (start 264.19 288.22) (end 264.19 286.51) (width 0.8) (layer "F.Cu") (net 3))
 (segment (start 214.9 238.25) (end 219.1 234.05) (width 1) (layer "F.Cu") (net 3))
 (segment (start 297.9 249.1) (end 308.3 249.1) (width 0.8) (layer "F.Cu") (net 3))
 (segment (start 251.6 279.7) (end 251.6 270.2) (width 1) (layer "F.Cu") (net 3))
 (segment (start 290.24 256.76) (end 297.9 249.1) (width 0.8) (layer "F.Cu") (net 3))
 (segment (start 214.9 242.6) (end 214.9 244.95) (width 1) (layer "F.Cu") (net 3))
 (segment (start 213.7 262.4) (end 207.4 256.1) (width 1) (layer "F.Cu") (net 3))
 (segment (start 219.1 234.05) (end 219.1 224.18) (width 1) (layer "F.Cu") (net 3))
 (segment (start 207.4 235.88) (end 219.1 224.18) (width 1) (layer "F.Cu") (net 3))
 (segment (start 301.42375 273) (end 307.02375 267.4) (width 1) (layer "F.Cu") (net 1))
 (segment (start 243.7 267.7) (end 246.9525 270.9525) (width 1) (layer "F.Cu") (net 1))
 (segment (start 223.874 215.474) (end 216.626 215.474) (width 1) (layer "F.Cu") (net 1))
 (segment (start 337.4 264.4) (end 337.4 233.7) (width 1) (layer "F.Cu") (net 1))
 (segment (start 334.4 267.4) (end 337.4 264.4) (width 1) (layer "F.Cu") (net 1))
 (segment (start 337.4 233.7) (end 319.3 215.6) (width 1) (layer "F.Cu") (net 1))
 (segment (start 224 215.6) (end 223.874 215.474) (width 1) (layer "F.Cu") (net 1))
 (segment (start 246.9525 270.9525) (end 246.9525 273) (width 1) (layer "F.Cu") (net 1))
 (segment (start 211.7 267.7) (end 243.7 267.7) (width 1) (layer "F.Cu") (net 1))
 (segment (start 319.3 215.6) (end 224 215.6) (width 1) (layer "F.Cu") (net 1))
 (segment (start 307.02375 267.4) (end 334.4 267.4) (width 1) (layer "F.Cu") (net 1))
 (segment (start 216.626 215.474) (end 204.5 227.6) (width 1) (layer "F.Cu") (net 1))
 (segment (start 204.5 260.5) (end 211.7 267.7) (width 1) (layer "F.Cu") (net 1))
 (segment (start 204.5 227.6) (end 204.5 260.5) (width 1) (layer "F.Cu") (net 1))
 (segment (start 269.27 265.17) (end 264.84 260.74) (width 0.8) (layer "F.Cu") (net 29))
 (segment (start 269.27 272.98) (end 269.27 265.17) (width 0.8) (layer "F.Cu") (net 29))
 (segment (start 264.84 260.74) (end 264.84 257.24) (width 0.8) (layer "F.Cu") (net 29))
 (segment (start 271.81 272.98) (end 271.81 265.31) (width 0.8) (layer "F.Cu") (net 28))
 (segment (start 271.81 265.31) (end 267.4 260.9) (width 0.8) (layer "F.Cu") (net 28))
 (segment (start 267.4 257.26) (end 267.38 257.24) (width 0.8) (layer "F.Cu") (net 28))
 (segment (start 267.4 260.9) (end 267.4 257.26) (width 0.8) (layer "F.Cu") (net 28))
 (segment (start 316.74 245.96) (end 316.74 236.8) (width 1) (layer "F.Cu") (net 4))
 (segment (start 292.78 257.24) (end 305.46 257.24) (width 1) (layer "F.Cu") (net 4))
 (segment (start 305.46 257.24) (end 316.74 245.96) (width 1) (layer "F.Cu") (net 4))
 (segment (start 261.65 288.22) (end 261.65 283.85) (width 1) (layer "F.Cu") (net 4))
 (segment (start 313.75875 279.1) (end 316.17625 276.6825) (width 1) (layer "F.Cu") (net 4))
 (segment (start 259.76 224.74) (end 259.76 226.8) (width 0.8) (layer "F.Cu") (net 4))
 (segment (start 263.2 221.3) (end 259.76 224.74) (width 0.8) (layer "F.Cu") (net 4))
 (segment (start 249.6 239.3) (end 249.6 242) (width 0.8) (layer "F.Cu") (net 4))
 (segment (start 316.17625 276.6825) (end 316.17625 273) (width 1) (layer "F.Cu") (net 4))
 (segment (start 282.62 226.8) (end 282.62 224.82) (width 0.8) (layer "F.Cu") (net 4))
 (segment (start 282.62 224.82) (end 279.1 221.3) (width 0.8) (layer "F.Cu") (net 4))
 (segment (start 261.65 283.85) (end 266.4 279.1) (width 1) (layer "F.Cu") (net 4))
 (segment (start 292.7 279.1) (end 292.78 257.24) (width 1) (layer "F.Cu") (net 4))
 (segment (start 279.1 221.3) (end 263.2 221.3) (width 0.8) (layer "F.Cu") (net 4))
 (segment (start 259.76 229.14) (end 249.6 239.3) (width 0.8) (layer "F.Cu") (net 4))
 (segment (start 259.76 226.8) (end 259.76 229.14) (width 0.8) (layer "F.Cu") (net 4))
 (segment (start 266.4 279.1) (end 313.75875 279.1) (width 1) (layer "F.Cu") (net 4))
 (segment (start 277.54 257.24) (end 277.54 259.96) (width 0.8) (layer "F.Cu") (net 27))
 (segment (start 277.5 260) (end 277.5 267.1) (width 0.8) (layer "F.Cu") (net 27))
 (segment (start 274.35 270.25) (end 274.35 272.98) (width 0.8) (layer "F.Cu") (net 27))
 (segment (start 277.5 267.1) (end 274.35 270.25) (width 0.8) (layer "F.Cu") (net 27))
 (segment (start 277.54 259.96) (end 277.5 260) (width 0.8) (layer "F.Cu") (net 27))
 (segment (start 264.19 266.99) (end 259.76 262.56) (width 0.8) (layer "F.Cu") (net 31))
 (segment (start 259.76 262.56) (end 259.76 257.24) (width 0.8) (layer "F.Cu") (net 31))
 (segment (start 264.19 272.98) (end 264.19 266.99) (width 0.8) (layer "F.Cu") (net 31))
 (segment (start 262.3 261.5) (end 262.3 257.24) (width 0.8) (layer "F.Cu") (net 30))
 (segment (start 266.73 272.98) (end 266.73 265.93) (width 0.8) (layer "F.Cu") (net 30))
 (segment (start 266.73 265.93) (end 262.3 261.5) (width 0.8) (layer "F.Cu") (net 30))
 (segment (start 230.22 288.22) (end 259.11 288.22) (width 1) (layer "F.Cu") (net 26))
 (segment (start 229.2 273) (end 227.1 275.1) (width 1) (layer "F.Cu") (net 26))
 (segment (start 232.2 273) (end 229.2 273) (width 1) (layer "F.Cu") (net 26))
 (segment (start 227.1 285.1) (end 230.22 288.22) (width 1) (layer "F.Cu") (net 26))
 (segment (start 227.1 275.1) (end 227.1 285.1) (width 1) (layer "F.Cu") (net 26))
 (segment (start 261.65 272.98) (end 261.65 267.85) (width 0.8) (layer "F.Cu") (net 32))
 (segment (start 257.22 263.42) (end 257.22 257.24) (width 0.8) (layer "F.Cu") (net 32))
 (segment (start 261.65 267.85) (end 257.22 263.42) (width 0.8) (layer "F.Cu") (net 32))
 (segment (start 252.14 257.24) (end 252.14 252.34) (width 0.8) (layer "F.Cu") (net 9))
 (segment (start 243.9 244.1) (end 239.4 244.1) (width 0.8) (layer "F.Cu") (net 9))
 (segment (start 252.14 252.34) (end 243.9 244.1) (width 0.8) (layer "F.Cu") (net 9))
 (segment (start 229.35 234.05) (end 224.1 234.05) (width 0.8) (layer "F.Cu") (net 9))
 (segment (start 239.4 244.1) (end 229.35 234.05) (width 0.8) (layer "F.Cu") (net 9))
 (segment (start 309.7 227.3) (end 316.4 227.3) (width 0.8) (layer "F.Cu") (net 38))
 (segment (start 321.82 232.72) (end 321.82 236.8) (width 0.8) (layer "F.Cu") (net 38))
 (segment (start 280.08 256.92) (end 309.7 227.3) (width 0.8) (layer "F.Cu") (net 38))
 (segment (start 280.08 257.24) (end 280.08 256.92) (width 0.8) (layer "F.Cu") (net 38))
 (segment (start 316.4 227.3) (end 321.82 232.72) (width 0.8) (layer "F.Cu") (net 38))
 (segment (start 241.75 249.15) (end 224.1 249.15) (width 0.8) (layer "F.Cu") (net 25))
 (segment (start 247.06 257.24) (end 247.06 254.46) (width 0.8) (layer "F.Cu") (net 25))
 (segment (start 247.06 254.46) (end 241.75 249.15) (width 0.8) (layer "F.Cu") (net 25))
 (segment (start 209.9 249) (end 209.9 242.6) (width 0.8) (layer "F.Cu") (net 8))
 (segment (start 244.52 257.24) (end 218.14 257.24) (width 0.8) (layer "F.Cu") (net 8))
 (segment (start 218.14 257.24) (end 209.9 249) (width 0.8) (layer "F.Cu") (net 8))
 (segment (start 242.8 246.7) (end 237.4 246.7) (width 0.8) (layer "F.Cu") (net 33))
 (segment (start 249.6 257.24) (end 249.6 253.5) (width 0.8) (layer "F.Cu") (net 33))
 (segment (start 237.4 246.7) (end 233.2 242.5) (width 0.8) (layer "F.Cu") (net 33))
 (segment (start 249.6 253.5) (end 242.8 246.7) (width 0.8) (layer "F.Cu") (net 33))
 (segment (start 282.62 257.24) (end 282.62 256.98) (width 0.8) (layer "F.Cu") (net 39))
 (segment (start 306 233.6) (end 316.08 233.6) (width 0.8) (layer "F.Cu") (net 39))
 (segment (start 282.62 256.98) (end 306 233.6) (width 0.8) (layer "F.Cu") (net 39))
 (segment (start 316.08 233.6) (end 319.28 236.8) (width 0.8) (layer "F.Cu") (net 39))
 (segment (start 269.27 294.03) (end 269.27 288.22) (width 1) (layer "F.Cu") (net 7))
 (segment (start 222.14 289.34) (end 228.78 295.98) (width 1) (layer "F.Cu") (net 7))
 (segment (start 218.6 289.34) (end 222.14 289.34) (width 1) (layer "F.Cu") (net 7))
 (segment (start 267.32 295.98) (end 269.27 294.03) (width 1) (layer "F.Cu") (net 7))
 (segment (start 228.78 295.98) (end 267.32 295.98) (width 1) (layer "F.Cu") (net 7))
 (segment (start 274.2 263.6) (end 272.46 261.86) (width 0.8) (layer "F.Cu") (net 36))
 (segment (start 272.46 261.86) (end 272.46 257.24) (width 0.8) (layer "F.Cu") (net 36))
 (segment (start 274.5 263.6) (end 274.2 263.6) (width 0.8) (layer "F.Cu") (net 36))
 (segment (start 259.11 272.98) (end 255.9 269.77) (width 0.8) (layer "F.Cu") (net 10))
 (segment (start 255.9 269.77) (end 255.9 267.9) (width 0.8) (layer "F.Cu") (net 10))
 (segment (start 269.92 242) (end 269.92 226.8) (width 0.8) (layer "F.Cu") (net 51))
 (segment (start 275 242) (end 275 226.8) (width 0.8) (layer "F.Cu") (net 53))
 (segment (start 277.54 226.8) (end 277.54 242) (width 0.8) (layer "F.Cu") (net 54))
 (segment (start 264.84 242) (end 264.84 226.8) (width 0.8) (layer "F.Cu") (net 49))
 (segment (start 267.38 242) (end 267.38 226.8) (width 0.8) (layer "F.Cu") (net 50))
 (segment (start 262.3 226.8) (end 262.3 242) (width 0.8) (layer "F.Cu") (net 48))
 (segment (start 280.08 242) (end 280.08 226.8) (width 0.8) (layer "F.Cu") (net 55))
 (segment (start 257.22 226.8) (end 247.06 236.96) (width 0.8) (layer "F.Cu") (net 43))
 (segment (start 247.06 236.96) (end 247.06 242) (width 0.8) (layer "F.Cu") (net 43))
 (segment (start 272.46 226.8) (end 272.46 242) (width 0.8) (layer "F.Cu") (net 52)))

